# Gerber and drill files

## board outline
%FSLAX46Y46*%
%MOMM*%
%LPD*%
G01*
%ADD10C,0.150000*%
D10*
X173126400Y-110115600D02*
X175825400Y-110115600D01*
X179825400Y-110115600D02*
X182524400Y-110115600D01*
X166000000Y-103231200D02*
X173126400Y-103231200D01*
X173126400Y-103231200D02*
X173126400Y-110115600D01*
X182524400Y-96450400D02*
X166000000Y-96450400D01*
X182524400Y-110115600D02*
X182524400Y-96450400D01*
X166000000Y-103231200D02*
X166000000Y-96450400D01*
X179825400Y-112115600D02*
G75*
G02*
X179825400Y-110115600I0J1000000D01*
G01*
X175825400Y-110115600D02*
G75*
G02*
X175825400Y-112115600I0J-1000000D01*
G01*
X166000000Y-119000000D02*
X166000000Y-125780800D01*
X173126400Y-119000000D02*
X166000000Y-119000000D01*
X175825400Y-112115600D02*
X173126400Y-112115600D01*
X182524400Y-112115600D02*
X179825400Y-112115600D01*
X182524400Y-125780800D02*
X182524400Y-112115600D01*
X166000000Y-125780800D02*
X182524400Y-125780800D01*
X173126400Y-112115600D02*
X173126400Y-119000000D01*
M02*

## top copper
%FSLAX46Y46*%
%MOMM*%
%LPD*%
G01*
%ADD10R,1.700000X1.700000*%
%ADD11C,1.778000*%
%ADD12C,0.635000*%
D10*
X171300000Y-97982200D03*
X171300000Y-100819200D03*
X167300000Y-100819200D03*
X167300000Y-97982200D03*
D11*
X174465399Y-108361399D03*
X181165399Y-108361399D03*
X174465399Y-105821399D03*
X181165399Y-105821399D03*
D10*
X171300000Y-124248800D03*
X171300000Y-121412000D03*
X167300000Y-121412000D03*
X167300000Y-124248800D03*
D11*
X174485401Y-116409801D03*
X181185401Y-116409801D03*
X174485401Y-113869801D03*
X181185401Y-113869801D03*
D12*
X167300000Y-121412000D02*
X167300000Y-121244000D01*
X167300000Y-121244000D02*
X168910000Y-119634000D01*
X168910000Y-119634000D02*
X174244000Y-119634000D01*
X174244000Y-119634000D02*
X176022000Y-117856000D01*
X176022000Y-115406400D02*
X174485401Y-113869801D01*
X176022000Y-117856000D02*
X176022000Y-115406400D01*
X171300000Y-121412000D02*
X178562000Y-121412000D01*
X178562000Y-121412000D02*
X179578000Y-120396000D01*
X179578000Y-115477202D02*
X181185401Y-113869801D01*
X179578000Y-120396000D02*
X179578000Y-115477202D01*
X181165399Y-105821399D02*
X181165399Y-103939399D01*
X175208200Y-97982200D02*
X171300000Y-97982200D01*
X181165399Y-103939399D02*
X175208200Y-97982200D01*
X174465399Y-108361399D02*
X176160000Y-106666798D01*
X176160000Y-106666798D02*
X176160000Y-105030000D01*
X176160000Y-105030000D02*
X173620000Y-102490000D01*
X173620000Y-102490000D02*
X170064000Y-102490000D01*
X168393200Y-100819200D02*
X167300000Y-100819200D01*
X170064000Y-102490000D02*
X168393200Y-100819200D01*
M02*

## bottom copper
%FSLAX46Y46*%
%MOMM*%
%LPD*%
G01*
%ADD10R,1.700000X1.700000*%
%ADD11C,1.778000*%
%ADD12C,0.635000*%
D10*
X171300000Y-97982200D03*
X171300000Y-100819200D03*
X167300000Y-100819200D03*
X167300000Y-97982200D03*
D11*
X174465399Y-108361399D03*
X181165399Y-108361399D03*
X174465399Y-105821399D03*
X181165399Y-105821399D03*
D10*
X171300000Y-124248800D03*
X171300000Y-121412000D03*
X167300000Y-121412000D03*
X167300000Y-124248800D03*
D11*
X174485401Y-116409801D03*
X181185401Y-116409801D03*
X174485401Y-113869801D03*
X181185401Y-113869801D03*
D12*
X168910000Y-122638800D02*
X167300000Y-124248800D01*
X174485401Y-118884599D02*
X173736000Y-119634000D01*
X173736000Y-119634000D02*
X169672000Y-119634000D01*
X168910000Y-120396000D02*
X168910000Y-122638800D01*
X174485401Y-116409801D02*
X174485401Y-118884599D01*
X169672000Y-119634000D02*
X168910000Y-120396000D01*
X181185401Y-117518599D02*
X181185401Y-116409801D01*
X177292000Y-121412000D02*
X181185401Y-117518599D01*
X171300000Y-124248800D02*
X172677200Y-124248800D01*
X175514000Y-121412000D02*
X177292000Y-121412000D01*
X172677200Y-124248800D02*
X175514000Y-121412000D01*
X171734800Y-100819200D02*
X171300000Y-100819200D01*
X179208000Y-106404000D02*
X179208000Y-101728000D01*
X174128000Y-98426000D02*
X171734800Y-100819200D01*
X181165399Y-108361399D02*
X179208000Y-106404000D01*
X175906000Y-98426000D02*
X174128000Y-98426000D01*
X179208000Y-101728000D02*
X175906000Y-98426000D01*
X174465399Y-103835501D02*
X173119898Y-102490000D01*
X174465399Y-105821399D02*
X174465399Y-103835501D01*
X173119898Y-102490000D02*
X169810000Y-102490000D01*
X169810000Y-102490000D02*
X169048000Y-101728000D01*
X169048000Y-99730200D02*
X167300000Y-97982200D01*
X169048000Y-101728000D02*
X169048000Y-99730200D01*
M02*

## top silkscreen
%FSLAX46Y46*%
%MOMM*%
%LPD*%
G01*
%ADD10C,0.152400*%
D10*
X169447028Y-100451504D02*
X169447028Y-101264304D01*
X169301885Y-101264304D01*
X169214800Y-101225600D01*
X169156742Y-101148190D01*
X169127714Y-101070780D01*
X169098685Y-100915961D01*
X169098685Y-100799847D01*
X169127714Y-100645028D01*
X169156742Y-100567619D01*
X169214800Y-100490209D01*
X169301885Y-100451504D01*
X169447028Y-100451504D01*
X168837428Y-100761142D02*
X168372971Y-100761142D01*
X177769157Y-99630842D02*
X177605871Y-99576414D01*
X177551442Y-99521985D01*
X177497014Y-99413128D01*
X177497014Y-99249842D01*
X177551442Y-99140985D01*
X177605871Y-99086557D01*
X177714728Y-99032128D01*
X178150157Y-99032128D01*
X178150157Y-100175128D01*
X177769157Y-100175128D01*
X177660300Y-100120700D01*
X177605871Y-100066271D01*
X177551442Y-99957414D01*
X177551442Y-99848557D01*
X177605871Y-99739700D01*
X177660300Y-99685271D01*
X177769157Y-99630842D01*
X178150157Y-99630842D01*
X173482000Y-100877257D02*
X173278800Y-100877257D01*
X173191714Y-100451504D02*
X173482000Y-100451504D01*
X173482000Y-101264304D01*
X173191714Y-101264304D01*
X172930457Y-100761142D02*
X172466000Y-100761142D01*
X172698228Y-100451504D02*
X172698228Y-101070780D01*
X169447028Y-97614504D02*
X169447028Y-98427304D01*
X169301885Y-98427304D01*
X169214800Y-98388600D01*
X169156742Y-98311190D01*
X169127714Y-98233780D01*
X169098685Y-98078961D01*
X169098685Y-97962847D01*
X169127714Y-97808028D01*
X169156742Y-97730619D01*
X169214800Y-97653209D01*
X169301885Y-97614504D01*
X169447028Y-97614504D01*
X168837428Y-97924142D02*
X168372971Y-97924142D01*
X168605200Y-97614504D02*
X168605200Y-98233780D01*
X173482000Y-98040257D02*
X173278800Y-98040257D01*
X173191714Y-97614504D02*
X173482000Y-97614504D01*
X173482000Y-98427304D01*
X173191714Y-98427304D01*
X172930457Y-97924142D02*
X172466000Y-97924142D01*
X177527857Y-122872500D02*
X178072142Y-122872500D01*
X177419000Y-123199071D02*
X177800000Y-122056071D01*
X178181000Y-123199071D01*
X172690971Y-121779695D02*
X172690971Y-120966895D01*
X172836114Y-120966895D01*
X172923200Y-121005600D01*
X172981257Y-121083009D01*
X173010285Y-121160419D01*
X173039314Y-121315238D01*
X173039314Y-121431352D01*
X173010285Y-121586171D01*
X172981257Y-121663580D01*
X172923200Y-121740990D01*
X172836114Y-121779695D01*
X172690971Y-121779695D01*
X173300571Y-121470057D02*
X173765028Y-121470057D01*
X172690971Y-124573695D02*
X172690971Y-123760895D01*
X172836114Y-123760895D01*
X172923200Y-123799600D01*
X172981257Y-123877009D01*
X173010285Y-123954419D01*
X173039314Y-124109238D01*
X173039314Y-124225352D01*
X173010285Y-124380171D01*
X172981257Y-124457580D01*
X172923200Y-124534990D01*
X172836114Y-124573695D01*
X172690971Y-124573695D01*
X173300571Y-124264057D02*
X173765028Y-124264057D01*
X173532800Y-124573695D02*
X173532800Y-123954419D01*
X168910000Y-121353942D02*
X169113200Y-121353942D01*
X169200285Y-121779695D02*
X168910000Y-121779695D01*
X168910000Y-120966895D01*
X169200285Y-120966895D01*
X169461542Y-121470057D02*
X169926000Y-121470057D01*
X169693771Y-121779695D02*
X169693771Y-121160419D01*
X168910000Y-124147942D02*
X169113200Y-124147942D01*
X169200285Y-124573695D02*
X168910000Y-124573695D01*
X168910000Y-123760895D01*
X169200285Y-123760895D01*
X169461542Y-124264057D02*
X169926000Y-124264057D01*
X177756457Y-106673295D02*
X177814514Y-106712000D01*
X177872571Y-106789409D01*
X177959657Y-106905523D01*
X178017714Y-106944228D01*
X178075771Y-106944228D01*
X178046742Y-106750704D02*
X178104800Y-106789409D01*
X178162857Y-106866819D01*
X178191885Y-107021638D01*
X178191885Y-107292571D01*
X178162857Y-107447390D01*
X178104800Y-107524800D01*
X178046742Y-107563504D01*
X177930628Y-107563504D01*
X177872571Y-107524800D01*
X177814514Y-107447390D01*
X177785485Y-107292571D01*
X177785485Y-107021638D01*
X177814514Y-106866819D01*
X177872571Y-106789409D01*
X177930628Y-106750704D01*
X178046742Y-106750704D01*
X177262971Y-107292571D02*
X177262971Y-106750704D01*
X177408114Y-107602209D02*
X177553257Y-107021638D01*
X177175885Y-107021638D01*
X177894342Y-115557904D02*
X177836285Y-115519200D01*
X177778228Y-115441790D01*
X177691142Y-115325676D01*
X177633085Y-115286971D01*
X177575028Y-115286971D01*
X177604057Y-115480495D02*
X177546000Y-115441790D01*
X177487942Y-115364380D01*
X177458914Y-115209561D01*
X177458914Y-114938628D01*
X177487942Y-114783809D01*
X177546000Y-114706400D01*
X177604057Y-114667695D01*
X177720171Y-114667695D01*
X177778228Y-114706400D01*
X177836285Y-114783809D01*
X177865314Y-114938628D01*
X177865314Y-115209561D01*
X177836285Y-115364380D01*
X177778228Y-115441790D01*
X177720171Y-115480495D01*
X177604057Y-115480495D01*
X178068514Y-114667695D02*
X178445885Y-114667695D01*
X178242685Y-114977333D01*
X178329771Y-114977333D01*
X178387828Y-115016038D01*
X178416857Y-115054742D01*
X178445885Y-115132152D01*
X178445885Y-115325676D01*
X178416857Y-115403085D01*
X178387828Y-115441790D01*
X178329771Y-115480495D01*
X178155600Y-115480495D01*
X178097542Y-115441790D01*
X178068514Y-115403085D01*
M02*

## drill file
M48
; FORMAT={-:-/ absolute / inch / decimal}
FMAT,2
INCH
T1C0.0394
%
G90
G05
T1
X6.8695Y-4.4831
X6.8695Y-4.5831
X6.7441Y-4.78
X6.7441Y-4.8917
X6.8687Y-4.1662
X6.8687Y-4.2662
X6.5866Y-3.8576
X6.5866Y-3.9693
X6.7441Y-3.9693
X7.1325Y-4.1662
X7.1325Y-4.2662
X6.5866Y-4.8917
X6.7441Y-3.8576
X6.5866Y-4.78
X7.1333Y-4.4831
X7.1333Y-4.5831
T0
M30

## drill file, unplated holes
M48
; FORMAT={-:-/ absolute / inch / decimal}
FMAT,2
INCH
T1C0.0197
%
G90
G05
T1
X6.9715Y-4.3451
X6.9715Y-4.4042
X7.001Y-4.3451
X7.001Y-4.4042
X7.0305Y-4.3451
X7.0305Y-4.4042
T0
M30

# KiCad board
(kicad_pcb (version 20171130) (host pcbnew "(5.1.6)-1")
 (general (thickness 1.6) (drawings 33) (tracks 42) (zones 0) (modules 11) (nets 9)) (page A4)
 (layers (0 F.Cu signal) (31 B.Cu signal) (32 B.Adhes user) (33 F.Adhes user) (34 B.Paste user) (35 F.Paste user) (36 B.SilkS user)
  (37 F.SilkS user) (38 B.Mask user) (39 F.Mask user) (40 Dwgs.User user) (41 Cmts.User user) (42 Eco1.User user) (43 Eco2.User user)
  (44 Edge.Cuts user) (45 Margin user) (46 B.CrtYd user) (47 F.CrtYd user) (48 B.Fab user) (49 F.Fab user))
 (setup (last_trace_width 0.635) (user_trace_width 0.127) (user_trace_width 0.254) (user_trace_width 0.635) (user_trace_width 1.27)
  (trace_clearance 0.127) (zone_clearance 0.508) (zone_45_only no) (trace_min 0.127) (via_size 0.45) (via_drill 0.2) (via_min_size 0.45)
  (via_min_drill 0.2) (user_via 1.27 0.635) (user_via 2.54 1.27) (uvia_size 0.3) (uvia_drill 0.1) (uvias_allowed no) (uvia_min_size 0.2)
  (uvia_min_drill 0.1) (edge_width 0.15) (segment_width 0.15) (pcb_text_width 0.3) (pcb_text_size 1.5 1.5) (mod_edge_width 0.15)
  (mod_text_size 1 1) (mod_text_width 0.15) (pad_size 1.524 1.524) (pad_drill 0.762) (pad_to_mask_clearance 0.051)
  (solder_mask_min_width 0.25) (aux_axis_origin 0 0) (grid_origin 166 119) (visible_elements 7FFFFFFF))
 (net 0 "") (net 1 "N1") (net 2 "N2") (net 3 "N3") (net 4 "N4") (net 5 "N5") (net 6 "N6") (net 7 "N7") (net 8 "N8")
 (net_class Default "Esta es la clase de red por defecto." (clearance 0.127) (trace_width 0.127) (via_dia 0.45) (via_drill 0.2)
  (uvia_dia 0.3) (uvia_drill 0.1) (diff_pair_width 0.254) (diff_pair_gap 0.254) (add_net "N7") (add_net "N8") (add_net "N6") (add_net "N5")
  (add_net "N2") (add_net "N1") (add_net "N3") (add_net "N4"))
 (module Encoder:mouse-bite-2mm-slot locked (layer F.Cu) (at 177.8254 111.1156)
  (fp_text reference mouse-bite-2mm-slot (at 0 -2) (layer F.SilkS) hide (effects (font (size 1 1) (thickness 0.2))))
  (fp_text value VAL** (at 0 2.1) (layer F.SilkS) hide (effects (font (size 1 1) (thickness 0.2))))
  (pad "" np_thru_hole circle (at 0.75 0.75) (size 0.5 0.5) (drill 0.5) (layers *.Cu *.Mask))
  (pad "" np_thru_hole circle (at -0.75 0.75) (size 0.5 0.5) (drill 0.5) (layers *.Cu *.Mask))
  (pad "" np_thru_hole circle (at -0.75 -0.75) (size 0.5 0.5) (drill 0.5) (layers *.Cu *.Mask))
  (pad "" np_thru_hole circle (at 0.75 -0.75) (size 0.5 0.5) (drill 0.5) (layers *.Cu *.Mask))
  (pad "" np_thru_hole circle (at 0 0.75) (size 0.5 0.5) (drill 0.5) (layers *.Cu *.Mask))
  (pad "" np_thru_hole circle (at 0 -0.75) (size 0.5 0.5) (drill 0.5) (layers *.Cu *.Mask)))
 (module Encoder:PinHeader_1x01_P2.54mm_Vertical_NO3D (layer F.Cu) (at 171.3 97.9822 180)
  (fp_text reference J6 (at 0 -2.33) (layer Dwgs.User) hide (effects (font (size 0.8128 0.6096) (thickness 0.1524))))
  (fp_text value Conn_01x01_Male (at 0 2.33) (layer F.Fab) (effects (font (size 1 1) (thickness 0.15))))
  (pad 1 thru_hole rect (at 0 0 180) (size 1.7 1.7) (drill 1) (layers *.Cu *.Mask) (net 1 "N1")))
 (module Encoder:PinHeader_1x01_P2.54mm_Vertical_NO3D (layer F.Cu) (at 171.3 100.8192 180)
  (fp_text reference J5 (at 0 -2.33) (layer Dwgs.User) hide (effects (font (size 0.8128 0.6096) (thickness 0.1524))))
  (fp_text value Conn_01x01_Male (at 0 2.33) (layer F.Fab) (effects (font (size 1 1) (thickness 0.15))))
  (pad 1 thru_hole rect (at 0 0 180) (size 1.7 1.7) (drill 1) (layers *.Cu *.Mask) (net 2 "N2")))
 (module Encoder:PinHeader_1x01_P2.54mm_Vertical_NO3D (layer F.Cu) (at 167.3 100.8192 180)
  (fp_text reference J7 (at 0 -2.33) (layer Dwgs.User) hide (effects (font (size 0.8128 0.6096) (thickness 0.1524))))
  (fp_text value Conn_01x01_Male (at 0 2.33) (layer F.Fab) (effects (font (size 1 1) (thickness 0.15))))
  (pad 1 thru_hole rect (at 0 0 180) (size 1.7 1.7) (drill 1) (layers *.Cu *.Mask) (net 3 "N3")))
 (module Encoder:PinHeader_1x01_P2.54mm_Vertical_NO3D (layer F.Cu) (at 167.3 97.9822 180)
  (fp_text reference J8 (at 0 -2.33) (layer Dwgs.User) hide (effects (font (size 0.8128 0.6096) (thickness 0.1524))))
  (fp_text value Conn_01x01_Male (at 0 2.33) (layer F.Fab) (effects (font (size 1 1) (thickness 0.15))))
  (pad 1 thru_hole rect (at 0 0 180) (size 1.7 1.7) (drill 1) (layers *.Cu *.Mask) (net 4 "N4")))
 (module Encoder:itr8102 (layer F.Cu) (at 177.815399 107.091399 180)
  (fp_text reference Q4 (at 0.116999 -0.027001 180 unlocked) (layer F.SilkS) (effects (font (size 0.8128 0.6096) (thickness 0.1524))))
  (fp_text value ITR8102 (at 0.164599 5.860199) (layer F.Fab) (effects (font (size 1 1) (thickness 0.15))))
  (pad 4 thru_hole circle (at 3.35 -1.27 180) (size 1.778 1.778) (drill 1) (layers *.Cu *.Mask) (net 3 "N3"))
  (pad 1 thru_hole circle (at -3.35 -1.27 180) (size 1.778 1.778) (drill 1) (layers *.Cu *.Mask) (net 2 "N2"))
  (pad 3 thru_hole circle (at 3.35 1.27 180) (size 1.778 1.778) (drill 1) (layers *.Cu *.Mask) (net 4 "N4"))
  (pad 2 thru_hole circle (at -3.35 1.27 180) (size 1.778 1.778) (drill 1) (layers *.Cu *.Mask) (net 1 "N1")))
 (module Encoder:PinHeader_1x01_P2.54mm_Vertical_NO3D (layer F.Cu) (at 171.3 124.2488)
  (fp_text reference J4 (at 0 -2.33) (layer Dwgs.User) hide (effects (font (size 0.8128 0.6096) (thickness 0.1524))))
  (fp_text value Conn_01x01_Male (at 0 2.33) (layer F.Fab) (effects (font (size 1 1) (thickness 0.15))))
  (pad 1 thru_hole rect (at 0 0) (size 1.7 1.7) (drill 1) (layers *.Cu *.Mask) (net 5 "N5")))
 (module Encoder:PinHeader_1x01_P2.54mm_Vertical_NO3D (layer F.Cu) (at 171.3 121.412)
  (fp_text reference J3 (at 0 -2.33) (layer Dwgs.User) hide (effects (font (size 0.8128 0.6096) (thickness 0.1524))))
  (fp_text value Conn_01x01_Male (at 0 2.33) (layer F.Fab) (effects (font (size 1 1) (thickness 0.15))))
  (pad 1 thru_hole rect (at 0 0) (size 1.7 1.7) (drill 1) (layers *.Cu *.Mask) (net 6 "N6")))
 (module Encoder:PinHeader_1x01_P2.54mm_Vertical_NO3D (layer F.Cu) (at 167.3 121.412)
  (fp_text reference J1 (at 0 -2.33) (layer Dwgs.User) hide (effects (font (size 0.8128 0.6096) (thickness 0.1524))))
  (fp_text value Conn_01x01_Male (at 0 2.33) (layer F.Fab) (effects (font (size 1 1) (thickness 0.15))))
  (pad 1 thru_hole rect (at 0 0) (size 1.7 1.7) (drill 1) (layers *.Cu *.Mask) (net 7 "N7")))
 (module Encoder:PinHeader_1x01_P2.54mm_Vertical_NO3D (layer F.Cu) (at 167.3 124.2488)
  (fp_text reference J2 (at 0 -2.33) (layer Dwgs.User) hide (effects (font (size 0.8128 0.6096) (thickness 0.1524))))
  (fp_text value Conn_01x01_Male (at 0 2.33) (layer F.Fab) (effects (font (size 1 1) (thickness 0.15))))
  (pad 1 thru_hole rect (at 0 0) (size 1.7 1.7) (drill 1) (layers *.Cu *.Mask) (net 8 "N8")))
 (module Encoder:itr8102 (layer F.Cu) (at 177.835401 115.139801)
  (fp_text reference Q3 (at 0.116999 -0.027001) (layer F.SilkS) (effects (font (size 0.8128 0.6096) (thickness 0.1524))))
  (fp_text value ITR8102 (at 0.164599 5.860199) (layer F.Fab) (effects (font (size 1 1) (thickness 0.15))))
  (pad 2 thru_hole circle (at -3.35 1.27) (size 1.778 1.778) (drill 1) (layers *.Cu *.Mask) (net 8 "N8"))
  (pad 3 thru_hole circle (at 3.35 1.27) (size 1.778 1.778) (drill 1) (layers *.Cu *.Mask) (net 5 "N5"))
  (pad 1 thru_hole circle (at -3.35 -1.27) (size 1.778 1.778) (drill 1) (layers *.Cu *.Mask) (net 7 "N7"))
  (pad 4 thru_hole circle (at 3.35 -1.27) (size 1.778 1.778) (drill 1) (layers *.Cu *.Mask) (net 6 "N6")))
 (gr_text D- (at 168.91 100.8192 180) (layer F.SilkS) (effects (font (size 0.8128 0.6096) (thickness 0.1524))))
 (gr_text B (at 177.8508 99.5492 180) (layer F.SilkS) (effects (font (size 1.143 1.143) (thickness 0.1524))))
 (gr_line (start 173.1264 110.1156) (end 175.8254 110.1156) (layer Edge.Cuts) (width 0.15))
 (gr_line (start 179.8254 110.1156) (end 182.5244 110.1156) (layer Edge.Cuts) (width 0.15))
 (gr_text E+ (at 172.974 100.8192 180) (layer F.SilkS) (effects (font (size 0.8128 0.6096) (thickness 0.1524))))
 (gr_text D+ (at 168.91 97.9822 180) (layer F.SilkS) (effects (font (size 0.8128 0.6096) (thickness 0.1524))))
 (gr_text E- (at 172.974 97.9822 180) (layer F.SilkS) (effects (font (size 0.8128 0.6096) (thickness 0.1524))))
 (gr_line (start 166 103.2312) (end 173.1264 103.2312) (layer Edge.Cuts) (width 0.15))
 (gr_line (start 173.1264 103.2312) (end 173.1264 110.1156) (layer Edge.Cuts) (width 0.15))
 (gr_line (start 182.5244 96.4504) (end 166 96.4504) (layer Edge.Cuts) (width 0.15))
 (gr_line (start 182.5244 110.1156) (end 182.5244 96.4504) (layer Edge.Cuts) (width 0.15))
 (gr_line (start 166 103.2312) (end 166 96.4504) (layer Edge.Cuts) (width 0.15))
 (gr_arc (start 179.8254 111.1156) (end 179.8254 110.1156) (angle -180) (layer Edge.Cuts) (width 0.15))
 (gr_arc (start 175.8254 111.1156) (end 175.8254 112.1156) (angle -180) (layer Edge.Cuts) (width 0.15))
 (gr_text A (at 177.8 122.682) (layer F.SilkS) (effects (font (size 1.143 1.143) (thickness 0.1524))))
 (gr_line (start 166 119) (end 166 125.7808) (layer Edge.Cuts) (width 0.15))
 (gr_line (start 173.1264 119) (end 166 119) (layer Edge.Cuts) (width 0.15))
 (gr_line (start 175.8254 112.1156) (end 173.1264 112.1156) (layer Edge.Cuts) (width 0.15))
 (gr_line (start 182.5244 112.1156) (end 179.8254 112.1156) (layer Edge.Cuts) (width 0.15))
 (gr_line (start 182.5244 125.7808) (end 182.5244 112.1156) (layer Edge.Cuts) (width 0.15))
 (gr_line (start 166 125.7808) (end 182.5244 125.7808) (layer Edge.Cuts) (width 0.15))
 (gr_line (start 173.1264 112.1156) (end 173.1264 119) (layer Edge.Cuts) (width 0.15))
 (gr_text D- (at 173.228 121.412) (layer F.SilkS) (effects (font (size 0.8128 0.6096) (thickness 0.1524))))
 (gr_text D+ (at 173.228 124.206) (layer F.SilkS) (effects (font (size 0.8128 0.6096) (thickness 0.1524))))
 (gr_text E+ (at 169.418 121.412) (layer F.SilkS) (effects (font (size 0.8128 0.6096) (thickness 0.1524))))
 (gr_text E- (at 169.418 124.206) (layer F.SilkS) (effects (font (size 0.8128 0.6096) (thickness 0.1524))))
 (segment (start 167.3 121.412) (end 167.3 121.244) (width 0.635) (layer F.Cu) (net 7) (status 30))
 (segment (start 167.3 121.244) (end 168.91 119.634) (width 0.635) (layer F.Cu) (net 7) (status 10))
 (segment (start 168.91 119.634) (end 174.244 119.634) (width 0.635) (layer F.Cu) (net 7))
 (segment (start 174.244 119.634) (end 176.022 117.856) (width 0.635) (layer F.Cu) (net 7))
 (segment (start 176.022 115.4064) (end 174.485401 113.869801) (width 0.635) (layer F.Cu) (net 7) (status 20))
 (segment (start 176.022 117.856) (end 176.022 115.4064) (width 0.635) (layer F.Cu) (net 7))
 (segment (start 168.91 122.6388) (end 167.3 124.2488) (width 0.635) (layer B.Cu) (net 8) (status 20))
 (segment (start 174.485401 118.884599) (end 173.736 119.634) (width 0.635) (layer B.Cu) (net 8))
 (segment (start 173.736 119.634) (end 169.672 119.634) (width 0.635) (layer B.Cu) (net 8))
 (segment (start 168.91 120.396) (end 168.91 122.6388) (width 0.635) (layer B.Cu) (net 8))
 (segment (start 174.485401 116.409801) (end 174.485401 118.884599) (width 0.635) (layer B.Cu) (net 8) (status 10))
 (segment (start 169.672 119.634) (end 168.91 120.396) (width 0.635) (layer B.Cu) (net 8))
 (segment (start 171.3 121.412) (end 178.562 121.412) (width 0.635) (layer F.Cu) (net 6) (status 10))
 (segment (start 178.562 121.412) (end 179.578 120.396) (width 0.635) (layer F.Cu) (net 6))
 (segment (start 179.578 115.477202) (end 181.185401 113.869801) (width 0.635) (layer F.Cu) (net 6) (status 20))
 (segment (start 179.578 120.396) (end 179.578 115.477202) (width 0.635) (layer F.Cu) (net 6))
 (segment (start 181.185401 117.518599) (end 181.185401 116.409801) (width 0.635) (layer B.Cu) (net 5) (status 20))
 (segment (start 177.292 121.412) (end 181.185401 117.518599) (width 0.635) (layer B.Cu) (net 5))
 (segment (start 171.3 124.2488) (end 172.6772 124.2488) (width 0.635) (layer B.Cu) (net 5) (status 10))
 (segment (start 175.514 121.412) (end 177.292 121.412) (width 0.635) (layer B.Cu) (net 5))
 (segment (start 172.6772 124.2488) (end 175.514 121.412) (width 0.635) (layer B.Cu) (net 5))
 (segment (start 171.7348 100.8192) (end 171.3 100.8192) (width 0.635) (layer B.Cu) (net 2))
 (segment (start 179.208 106.404) (end 179.208 101.728) (width 0.635) (layer B.Cu) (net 2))
 (segment (start 174.128 98.426) (end 171.7348 100.8192) (width 0.635) (layer B.Cu) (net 2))
 (segment (start 181.165399 108.361399) (end 179.208 106.404) (width 0.635) (layer B.Cu) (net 2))
 (segment (start 175.906 98.426) (end 174.128 98.426) (width 0.635) (layer B.Cu) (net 2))
 (segment (start 179.208 101.728) (end 175.906 98.426) (width 0.635) (layer B.Cu) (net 2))
 (segment (start 181.165399 105.821399) (end 181.165399 103.939399) (width 0.635) (layer F.Cu) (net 1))
 (segment (start 175.2082 97.9822) (end 171.3 97.9822) (width 0.635) (layer F.Cu) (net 1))
 (segment (start 181.165399 103.939399) (end 175.2082 97.9822) (width 0.635) (layer F.Cu) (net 1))
 (segment (start 174.465399 108.361399) (end 176.16 106.666798) (width 0.635) (layer F.Cu) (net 3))
 (segment (start 176.16 106.666798) (end 176.16 105.03) (width 0.635) (layer F.Cu) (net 3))
 (segment (start 176.16 105.03) (end 173.62 102.49) (width 0.635) (layer F.Cu) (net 3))
 (segment (start 173.62 102.49) (end 170.064 102.49) (width 0.635) (layer F.Cu) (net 3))
 (segment (start 168.3932 100.8192) (end 167.3 100.8192) (width 0.635) (layer F.Cu) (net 3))
 (segment (start 170.064 102.49) (end 168.3932 100.8192) (width 0.635) (layer F.Cu) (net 3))
 (segment (start 174.465399 103.835501) (end 173.119898 102.49) (width 0.635) (layer B.Cu) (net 4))
 (segment (start 174.465399 105.821399) (end 174.465399 103.835501) (width 0.635) (layer B.Cu) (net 4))
 (segment (start 173.119898 102.49) (end 169.81 102.49) (width 0.635) (layer B.Cu) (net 4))
 (segment (start 169.81 102.49) (end 169.048 101.728) (width 0.635) (layer B.Cu) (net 4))
 (segment (start 169.048 99.7302) (end 167.3 97.9822) (width 0.635) (layer B.Cu) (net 4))
 (segment (start 169.048 101.728) (end 169.048 99.7302) (width 0.635) (layer B.Cu) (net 4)))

